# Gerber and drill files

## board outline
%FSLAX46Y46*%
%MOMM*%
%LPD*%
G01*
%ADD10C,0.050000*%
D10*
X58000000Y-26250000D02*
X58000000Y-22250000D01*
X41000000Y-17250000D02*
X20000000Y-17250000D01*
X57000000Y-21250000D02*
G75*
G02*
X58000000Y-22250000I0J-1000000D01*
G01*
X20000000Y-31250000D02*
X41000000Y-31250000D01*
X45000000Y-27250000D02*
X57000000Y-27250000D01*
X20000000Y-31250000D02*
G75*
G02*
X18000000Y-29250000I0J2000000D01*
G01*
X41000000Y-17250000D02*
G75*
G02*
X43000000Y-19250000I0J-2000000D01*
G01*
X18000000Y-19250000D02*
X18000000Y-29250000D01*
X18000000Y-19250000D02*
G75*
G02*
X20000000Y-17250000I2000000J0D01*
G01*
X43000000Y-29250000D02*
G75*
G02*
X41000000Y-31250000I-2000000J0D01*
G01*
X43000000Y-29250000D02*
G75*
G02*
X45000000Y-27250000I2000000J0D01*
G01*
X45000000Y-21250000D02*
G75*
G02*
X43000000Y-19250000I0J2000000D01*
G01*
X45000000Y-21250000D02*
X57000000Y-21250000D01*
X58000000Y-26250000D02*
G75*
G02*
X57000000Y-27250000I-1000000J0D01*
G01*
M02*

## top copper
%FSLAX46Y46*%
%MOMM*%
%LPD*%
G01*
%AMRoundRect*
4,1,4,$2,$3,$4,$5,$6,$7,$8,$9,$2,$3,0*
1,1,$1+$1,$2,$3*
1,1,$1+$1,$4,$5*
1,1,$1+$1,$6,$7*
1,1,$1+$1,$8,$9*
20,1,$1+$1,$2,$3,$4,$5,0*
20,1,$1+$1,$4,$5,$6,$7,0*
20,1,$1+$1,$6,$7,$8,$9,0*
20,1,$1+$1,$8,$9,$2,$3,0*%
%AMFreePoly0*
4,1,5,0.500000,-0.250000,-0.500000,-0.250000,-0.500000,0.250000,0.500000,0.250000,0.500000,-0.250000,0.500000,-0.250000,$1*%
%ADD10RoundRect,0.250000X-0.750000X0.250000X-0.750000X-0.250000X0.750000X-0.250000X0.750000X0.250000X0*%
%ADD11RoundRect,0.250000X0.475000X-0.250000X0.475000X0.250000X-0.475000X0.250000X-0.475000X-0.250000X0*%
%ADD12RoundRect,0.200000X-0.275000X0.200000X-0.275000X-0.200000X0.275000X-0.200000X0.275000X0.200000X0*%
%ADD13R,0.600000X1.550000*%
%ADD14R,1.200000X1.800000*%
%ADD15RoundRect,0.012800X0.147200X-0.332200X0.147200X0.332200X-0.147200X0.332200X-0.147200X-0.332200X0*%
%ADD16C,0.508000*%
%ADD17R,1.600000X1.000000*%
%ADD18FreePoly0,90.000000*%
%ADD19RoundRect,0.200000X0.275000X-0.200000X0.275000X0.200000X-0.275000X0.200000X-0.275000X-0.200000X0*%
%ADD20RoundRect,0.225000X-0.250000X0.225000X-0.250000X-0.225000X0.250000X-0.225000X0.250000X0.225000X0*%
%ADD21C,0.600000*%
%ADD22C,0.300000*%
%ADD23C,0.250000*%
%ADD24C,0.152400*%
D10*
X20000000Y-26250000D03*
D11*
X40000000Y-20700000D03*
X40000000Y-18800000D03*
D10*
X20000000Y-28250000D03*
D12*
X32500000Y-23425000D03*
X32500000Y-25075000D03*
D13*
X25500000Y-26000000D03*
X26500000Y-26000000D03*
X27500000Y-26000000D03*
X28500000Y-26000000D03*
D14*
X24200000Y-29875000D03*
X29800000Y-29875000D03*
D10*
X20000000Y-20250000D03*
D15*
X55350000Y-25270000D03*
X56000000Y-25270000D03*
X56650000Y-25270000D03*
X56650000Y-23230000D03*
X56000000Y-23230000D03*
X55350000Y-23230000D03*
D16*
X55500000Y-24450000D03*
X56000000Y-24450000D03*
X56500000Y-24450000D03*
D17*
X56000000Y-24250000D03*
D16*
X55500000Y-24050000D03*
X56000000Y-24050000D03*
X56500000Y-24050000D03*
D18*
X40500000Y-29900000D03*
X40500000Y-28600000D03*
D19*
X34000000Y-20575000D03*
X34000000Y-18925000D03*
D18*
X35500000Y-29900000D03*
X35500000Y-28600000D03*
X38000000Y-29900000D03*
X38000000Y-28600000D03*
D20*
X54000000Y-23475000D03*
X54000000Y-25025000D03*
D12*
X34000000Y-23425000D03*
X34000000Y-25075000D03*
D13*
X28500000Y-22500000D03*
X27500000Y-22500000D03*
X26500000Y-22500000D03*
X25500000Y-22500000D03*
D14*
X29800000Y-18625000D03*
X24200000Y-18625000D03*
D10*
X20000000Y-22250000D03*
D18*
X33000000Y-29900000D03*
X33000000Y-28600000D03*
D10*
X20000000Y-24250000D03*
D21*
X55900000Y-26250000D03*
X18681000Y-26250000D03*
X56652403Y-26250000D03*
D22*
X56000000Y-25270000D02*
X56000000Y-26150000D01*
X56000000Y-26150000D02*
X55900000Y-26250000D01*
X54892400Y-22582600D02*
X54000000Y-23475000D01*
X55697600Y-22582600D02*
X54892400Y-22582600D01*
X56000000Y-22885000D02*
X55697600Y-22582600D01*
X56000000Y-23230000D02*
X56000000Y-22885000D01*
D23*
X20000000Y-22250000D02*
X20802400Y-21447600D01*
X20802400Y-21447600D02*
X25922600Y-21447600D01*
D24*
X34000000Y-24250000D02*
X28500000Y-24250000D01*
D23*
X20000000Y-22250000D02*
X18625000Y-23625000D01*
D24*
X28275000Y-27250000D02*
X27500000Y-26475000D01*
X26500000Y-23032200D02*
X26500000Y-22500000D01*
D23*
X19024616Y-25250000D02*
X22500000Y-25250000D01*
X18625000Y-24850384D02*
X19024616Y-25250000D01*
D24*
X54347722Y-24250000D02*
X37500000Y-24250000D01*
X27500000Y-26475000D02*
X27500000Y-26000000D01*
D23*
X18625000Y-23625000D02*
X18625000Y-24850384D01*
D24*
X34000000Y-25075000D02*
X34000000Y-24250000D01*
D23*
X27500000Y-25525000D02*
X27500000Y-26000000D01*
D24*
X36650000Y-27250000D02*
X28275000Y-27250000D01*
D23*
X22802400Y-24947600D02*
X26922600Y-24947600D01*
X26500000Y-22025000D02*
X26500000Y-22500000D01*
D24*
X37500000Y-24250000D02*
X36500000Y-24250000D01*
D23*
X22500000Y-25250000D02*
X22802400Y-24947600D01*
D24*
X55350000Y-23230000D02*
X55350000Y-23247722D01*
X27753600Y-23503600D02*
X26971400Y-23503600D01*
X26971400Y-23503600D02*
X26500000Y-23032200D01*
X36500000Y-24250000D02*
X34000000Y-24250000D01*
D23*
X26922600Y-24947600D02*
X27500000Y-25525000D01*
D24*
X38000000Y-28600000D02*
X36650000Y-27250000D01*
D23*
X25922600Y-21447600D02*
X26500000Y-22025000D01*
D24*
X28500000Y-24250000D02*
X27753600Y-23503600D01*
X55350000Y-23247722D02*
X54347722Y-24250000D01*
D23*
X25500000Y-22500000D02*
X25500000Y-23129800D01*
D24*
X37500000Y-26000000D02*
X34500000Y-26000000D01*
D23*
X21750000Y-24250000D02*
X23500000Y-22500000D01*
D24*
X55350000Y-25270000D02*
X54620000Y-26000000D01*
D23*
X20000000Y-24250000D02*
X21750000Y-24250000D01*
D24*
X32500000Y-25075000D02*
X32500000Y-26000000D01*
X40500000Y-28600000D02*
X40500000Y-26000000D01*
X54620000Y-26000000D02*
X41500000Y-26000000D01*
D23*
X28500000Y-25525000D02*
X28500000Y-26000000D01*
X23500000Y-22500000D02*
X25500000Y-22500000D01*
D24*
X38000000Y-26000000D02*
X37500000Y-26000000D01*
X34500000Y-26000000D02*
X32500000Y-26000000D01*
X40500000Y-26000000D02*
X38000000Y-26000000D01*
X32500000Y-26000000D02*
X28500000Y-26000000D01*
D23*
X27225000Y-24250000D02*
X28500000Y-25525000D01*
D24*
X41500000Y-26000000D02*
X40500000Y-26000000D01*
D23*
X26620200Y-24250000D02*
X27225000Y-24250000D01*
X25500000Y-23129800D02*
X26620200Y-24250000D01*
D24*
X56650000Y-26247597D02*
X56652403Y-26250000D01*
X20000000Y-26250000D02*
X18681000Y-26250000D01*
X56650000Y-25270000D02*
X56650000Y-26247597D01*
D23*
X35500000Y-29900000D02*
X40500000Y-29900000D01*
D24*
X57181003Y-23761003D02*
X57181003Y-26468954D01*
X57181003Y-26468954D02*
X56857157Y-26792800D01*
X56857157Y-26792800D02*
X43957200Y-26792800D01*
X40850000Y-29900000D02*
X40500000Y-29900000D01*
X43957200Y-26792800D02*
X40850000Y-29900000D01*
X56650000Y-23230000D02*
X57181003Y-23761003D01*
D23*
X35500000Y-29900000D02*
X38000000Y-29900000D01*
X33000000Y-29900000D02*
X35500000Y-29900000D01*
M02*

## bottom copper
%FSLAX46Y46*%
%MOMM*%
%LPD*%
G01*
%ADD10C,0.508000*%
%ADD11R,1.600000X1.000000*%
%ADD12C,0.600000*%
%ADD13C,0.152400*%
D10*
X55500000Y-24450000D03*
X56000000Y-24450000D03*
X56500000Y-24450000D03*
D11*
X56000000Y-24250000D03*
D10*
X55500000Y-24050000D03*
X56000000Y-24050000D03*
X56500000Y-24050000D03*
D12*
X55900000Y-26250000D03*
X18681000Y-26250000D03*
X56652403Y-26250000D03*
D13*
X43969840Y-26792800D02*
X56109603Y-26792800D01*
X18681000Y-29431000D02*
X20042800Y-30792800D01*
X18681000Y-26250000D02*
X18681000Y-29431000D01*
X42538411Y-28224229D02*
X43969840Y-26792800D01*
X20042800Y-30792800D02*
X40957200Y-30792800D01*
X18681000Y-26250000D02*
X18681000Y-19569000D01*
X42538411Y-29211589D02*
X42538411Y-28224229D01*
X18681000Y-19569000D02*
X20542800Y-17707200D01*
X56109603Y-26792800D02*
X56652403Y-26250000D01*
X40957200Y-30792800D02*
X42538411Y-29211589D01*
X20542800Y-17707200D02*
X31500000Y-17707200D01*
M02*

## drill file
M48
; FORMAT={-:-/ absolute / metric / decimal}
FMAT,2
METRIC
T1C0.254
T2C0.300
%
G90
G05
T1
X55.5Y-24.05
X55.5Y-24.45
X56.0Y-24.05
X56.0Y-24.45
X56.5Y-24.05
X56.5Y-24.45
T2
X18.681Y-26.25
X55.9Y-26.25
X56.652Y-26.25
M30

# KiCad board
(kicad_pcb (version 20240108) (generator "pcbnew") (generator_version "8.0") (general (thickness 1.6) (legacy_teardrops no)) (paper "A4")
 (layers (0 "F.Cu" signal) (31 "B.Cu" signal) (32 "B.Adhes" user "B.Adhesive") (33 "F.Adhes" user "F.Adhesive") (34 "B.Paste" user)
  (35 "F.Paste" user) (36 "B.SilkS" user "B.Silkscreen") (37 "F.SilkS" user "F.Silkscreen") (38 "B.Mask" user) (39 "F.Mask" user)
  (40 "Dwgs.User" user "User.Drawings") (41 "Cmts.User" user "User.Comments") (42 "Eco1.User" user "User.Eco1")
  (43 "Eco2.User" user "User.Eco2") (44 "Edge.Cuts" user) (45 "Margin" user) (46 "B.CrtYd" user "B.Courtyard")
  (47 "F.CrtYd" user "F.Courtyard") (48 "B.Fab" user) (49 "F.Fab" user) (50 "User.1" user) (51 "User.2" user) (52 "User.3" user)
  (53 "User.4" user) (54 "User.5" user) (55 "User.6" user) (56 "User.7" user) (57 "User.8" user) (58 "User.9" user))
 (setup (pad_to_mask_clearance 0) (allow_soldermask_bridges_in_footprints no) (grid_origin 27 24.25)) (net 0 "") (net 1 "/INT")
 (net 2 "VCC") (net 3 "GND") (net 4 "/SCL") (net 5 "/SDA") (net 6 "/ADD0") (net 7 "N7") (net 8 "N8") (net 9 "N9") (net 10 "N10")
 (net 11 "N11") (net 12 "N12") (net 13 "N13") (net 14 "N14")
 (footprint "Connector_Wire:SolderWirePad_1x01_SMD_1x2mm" (layer "F.Cu") (at 20 26.25 -90)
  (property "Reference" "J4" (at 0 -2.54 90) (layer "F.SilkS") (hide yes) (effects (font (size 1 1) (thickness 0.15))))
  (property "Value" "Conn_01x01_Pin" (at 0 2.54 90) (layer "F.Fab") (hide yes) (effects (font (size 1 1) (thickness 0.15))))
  (pad "1" smd roundrect (at 0 0 270) (size 1 2) (layers "F.Cu" "F.Paste" "F.Mask") (roundrect_rratio 0.25) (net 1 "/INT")))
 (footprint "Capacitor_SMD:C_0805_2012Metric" (layer "F.Cu") (at 40 19.75 90)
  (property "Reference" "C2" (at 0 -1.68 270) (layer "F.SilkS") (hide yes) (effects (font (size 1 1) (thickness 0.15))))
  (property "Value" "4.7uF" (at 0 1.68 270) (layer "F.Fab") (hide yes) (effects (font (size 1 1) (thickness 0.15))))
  (pad "1" smd roundrect (at -0.95 0 90) (size 1 1.45) (layers "F.Cu" "F.Paste" "F.Mask") (roundrect_rratio 0.25) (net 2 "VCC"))
  (pad "2" smd roundrect (at 0.95 0 90) (size 1 1.45) (layers "F.Cu" "F.Paste" "F.Mask") (roundrect_rratio 0.25) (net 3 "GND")))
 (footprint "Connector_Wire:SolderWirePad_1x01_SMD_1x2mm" (layer "F.Cu") (at 20 28.25 -90)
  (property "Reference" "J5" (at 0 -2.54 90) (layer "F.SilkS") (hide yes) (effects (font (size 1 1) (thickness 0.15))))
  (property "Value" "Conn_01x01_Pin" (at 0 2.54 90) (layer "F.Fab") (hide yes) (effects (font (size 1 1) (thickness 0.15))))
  (pad "1" smd roundrect (at 0 0 270) (size 1 2) (layers "F.Cu" "F.Paste" "F.Mask") (roundrect_rratio 0.25) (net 3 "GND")))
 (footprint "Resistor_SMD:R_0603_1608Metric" (layer "F.Cu") (at 32.5 24.25 -90)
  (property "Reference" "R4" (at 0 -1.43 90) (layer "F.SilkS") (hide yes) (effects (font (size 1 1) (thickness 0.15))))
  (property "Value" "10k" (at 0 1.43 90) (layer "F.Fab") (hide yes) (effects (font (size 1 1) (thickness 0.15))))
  (pad "1" smd roundrect (at -0.825 0 270) (size 0.8 0.95) (layers "F.Cu" "F.Paste" "F.Mask") (roundrect_rratio 0.25) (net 2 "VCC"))
  (pad "2" smd roundrect (at 0.825 0 270) (size 0.8 0.95) (layers "F.Cu" "F.Paste" "F.Mask") (roundrect_rratio 0.25) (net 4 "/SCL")))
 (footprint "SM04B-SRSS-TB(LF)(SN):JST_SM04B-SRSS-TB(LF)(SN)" (layer "F.Cu") (at 27 26)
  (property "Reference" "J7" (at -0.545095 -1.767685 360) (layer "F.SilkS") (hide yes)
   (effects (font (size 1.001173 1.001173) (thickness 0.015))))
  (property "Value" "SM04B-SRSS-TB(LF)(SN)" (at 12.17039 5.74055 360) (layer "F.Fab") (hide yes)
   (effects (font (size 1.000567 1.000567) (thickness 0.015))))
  (pad "1" smd rect (at -1.5 0) (size 0.6 1.55) (layers "F.Cu" "F.Paste" "F.Mask") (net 3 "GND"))
  (pad "2" smd rect (at -0.5 0) (size 0.6 1.55) (layers "F.Cu" "F.Paste" "F.Mask") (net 2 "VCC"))
  (pad "3" smd rect (at 0.5 0) (size 0.6 1.55) (layers "F.Cu" "F.Paste" "F.Mask") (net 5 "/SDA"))
  (pad "4" smd rect (at 1.5 0) (size 0.6 1.55) (layers "F.Cu" "F.Paste" "F.Mask") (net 4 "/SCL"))
  (pad "S1" smd rect (at -2.8 3.875) (size 1.2 1.8) (layers "F.Cu" "F.Paste" "F.Mask") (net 3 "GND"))
  (pad "S2" smd rect (at 2.8 3.875) (size 1.2 1.8) (layers "F.Cu" "F.Paste" "F.Mask") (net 3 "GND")))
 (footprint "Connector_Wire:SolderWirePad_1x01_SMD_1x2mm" (layer "F.Cu") (at 20 20.25 -90)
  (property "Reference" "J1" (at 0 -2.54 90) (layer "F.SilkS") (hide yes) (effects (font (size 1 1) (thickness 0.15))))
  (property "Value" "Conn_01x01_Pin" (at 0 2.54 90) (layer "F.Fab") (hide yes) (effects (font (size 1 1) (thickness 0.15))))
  (pad "1" smd roundrect (at 0 0 270) (size 1 2) (layers "F.Cu" "F.Paste" "F.Mask") (roundrect_rratio 0.25) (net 2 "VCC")))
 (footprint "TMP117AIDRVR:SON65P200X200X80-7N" (layer "F.Cu") (at 56 24.25 90)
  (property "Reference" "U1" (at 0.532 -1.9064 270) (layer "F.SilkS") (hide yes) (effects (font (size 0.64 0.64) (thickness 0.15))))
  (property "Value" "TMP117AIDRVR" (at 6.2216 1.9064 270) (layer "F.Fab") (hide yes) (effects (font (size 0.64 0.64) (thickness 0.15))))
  (pad "1" smd roundrect (at -1.02 -0.65 90) (size 0.69 0.32) (layers "F.Cu" "F.Paste" "F.Mask") (roundrect_rratio 0.04) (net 4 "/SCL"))
  (pad "2" smd roundrect (at -1.02 0 90) (size 0.69 0.32) (layers "F.Cu" "F.Paste" "F.Mask") (roundrect_rratio 0.04) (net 3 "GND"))
  (pad "3" smd roundrect (at -1.02 0.65 90) (size 0.69 0.32) (layers "F.Cu" "F.Paste" "F.Mask") (roundrect_rratio 0.04) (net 1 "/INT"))
  (pad "4" smd roundrect (at 1.02 0.65 90) (size 0.69 0.32) (layers "F.Cu" "F.Paste" "F.Mask") (roundrect_rratio 0.04) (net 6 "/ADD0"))
  (pad "5" smd roundrect (at 1.02 0 90) (size 0.69 0.32) (layers "F.Cu" "F.Paste" "F.Mask") (roundrect_rratio 0.04) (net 2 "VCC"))
  (pad "6" smd roundrect (at 1.02 -0.65 90) (size 0.69 0.32) (layers "F.Cu" "F.Paste" "F.Mask") (roundrect_rratio 0.04) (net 5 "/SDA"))
  (pad "7" thru_hole circle (at -0.2 -0.5 180) (size 0.508 0.508) (drill 0.254) (layers "*.Cu" "*.Mask") (remove_unused_layers no)
   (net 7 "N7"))
  (pad "7" thru_hole circle (at -0.2 0 180) (size 0.508 0.508) (drill 0.254) (layers "*.Cu" "*.Mask") (remove_unused_layers no) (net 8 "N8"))
  (pad "7" thru_hole circle (at -0.2 0.5 180) (size 0.508 0.508) (drill 0.254) (layers "*.Cu" "*.Mask") (remove_unused_layers no)
   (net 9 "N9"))
  (pad "7" smd rect (at 0 0 180) (size 1.6 1) (layers "F.Cu" "F.Mask") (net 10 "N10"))
  (pad "7" smd rect (at 0 0 180) (size 1.6 1) (layers "B.Cu" "B.Mask") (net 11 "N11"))
  (pad "7" thru_hole circle (at 0.2 -0.5 180) (size 0.508 0.508) (drill 0.254) (layers "*.Cu" "*.Mask") (remove_unused_layers no)
   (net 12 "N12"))
  (pad "7" thru_hole circle (at 0.2 0 180) (size 0.508 0.508) (drill 0.254) (layers "*.Cu" "*.Mask") (remove_unused_layers no)
   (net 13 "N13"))
  (pad "7" thru_hole circle (at 0.2 0.5 180) (size 0.508 0.508) (drill 0.254) (layers "*.Cu" "*.Mask") (remove_unused_layers no)
   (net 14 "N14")))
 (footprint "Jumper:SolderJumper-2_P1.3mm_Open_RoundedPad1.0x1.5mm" (layer "F.Cu") (at 40.5 29.25 90)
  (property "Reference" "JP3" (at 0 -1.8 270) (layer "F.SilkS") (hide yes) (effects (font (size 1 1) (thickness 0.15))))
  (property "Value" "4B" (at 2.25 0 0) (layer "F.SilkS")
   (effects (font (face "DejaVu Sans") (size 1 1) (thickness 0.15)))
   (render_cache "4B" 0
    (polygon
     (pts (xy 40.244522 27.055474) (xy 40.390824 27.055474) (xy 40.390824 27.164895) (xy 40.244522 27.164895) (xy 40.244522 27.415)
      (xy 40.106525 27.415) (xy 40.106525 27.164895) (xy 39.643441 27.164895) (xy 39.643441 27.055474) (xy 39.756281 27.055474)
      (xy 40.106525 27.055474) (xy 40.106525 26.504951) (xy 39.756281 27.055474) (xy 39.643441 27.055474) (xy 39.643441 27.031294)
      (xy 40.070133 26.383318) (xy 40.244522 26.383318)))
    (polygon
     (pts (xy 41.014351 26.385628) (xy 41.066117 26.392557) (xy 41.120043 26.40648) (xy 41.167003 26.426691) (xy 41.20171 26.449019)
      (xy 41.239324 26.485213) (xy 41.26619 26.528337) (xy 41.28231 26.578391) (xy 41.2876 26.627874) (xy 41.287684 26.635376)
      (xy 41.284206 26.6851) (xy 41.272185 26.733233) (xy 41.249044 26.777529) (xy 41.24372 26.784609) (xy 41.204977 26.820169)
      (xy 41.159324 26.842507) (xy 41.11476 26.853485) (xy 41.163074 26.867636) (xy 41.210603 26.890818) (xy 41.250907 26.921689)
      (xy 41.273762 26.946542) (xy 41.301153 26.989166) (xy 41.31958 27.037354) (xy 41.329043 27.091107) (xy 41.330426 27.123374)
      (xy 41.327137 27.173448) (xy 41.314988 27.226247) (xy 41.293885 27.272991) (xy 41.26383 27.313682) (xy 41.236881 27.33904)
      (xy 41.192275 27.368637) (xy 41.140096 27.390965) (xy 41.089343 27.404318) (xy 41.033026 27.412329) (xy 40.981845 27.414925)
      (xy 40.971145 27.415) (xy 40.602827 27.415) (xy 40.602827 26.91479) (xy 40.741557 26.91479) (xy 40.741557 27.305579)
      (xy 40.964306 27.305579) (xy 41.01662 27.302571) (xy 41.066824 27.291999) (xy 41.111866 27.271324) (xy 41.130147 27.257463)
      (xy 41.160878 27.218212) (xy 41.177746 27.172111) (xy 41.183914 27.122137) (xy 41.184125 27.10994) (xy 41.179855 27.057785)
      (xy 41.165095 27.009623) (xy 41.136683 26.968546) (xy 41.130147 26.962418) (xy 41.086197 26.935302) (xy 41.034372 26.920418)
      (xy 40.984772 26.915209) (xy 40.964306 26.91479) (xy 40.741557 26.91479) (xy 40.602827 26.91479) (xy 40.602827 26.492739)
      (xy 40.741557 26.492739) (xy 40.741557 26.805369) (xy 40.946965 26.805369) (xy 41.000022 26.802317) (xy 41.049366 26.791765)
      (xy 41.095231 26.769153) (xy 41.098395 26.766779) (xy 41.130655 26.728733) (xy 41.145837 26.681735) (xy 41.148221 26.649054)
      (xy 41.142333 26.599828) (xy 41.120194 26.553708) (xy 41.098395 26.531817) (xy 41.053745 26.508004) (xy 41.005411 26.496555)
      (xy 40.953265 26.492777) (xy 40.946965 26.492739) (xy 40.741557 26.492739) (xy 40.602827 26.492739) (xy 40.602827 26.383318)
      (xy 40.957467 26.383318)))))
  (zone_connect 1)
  (pad "1" smd custom (at -0.65 0 90) (size 1 0.5) (layers "F.Cu" "F.Mask") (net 6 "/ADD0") (zone_connect 2) (thermal_bridge_angle 45)
   (options (clearance outline) (anchor rect)) (primitives))
  (pad "2" smd custom (at 0.65 0 90) (size 1 0.5) (layers "F.Cu" "F.Mask") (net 4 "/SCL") (zone_connect 2) (thermal_bridge_angle 45)
   (options (clearance outline) (anchor rect)) (primitives)))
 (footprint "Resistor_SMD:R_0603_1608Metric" (layer "F.Cu") (at 34 19.75 90)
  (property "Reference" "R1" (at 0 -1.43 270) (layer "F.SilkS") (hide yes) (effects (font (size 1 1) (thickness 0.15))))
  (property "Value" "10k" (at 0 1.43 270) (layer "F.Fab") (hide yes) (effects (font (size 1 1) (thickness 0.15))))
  (pad "1" smd roundrect (at -0.825 0 90) (size 0.8 0.95) (layers "F.Cu" "F.Paste" "F.Mask") (roundrect_rratio 0.25) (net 2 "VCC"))
  (pad "2" smd roundrect (at 0.825 0 90) (size 0.8 0.95) (layers "F.Cu" "F.Paste" "F.Mask") (roundrect_rratio 0.25) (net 1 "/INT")))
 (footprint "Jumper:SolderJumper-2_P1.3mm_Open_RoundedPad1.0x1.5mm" (layer "F.Cu") (at 35.5 29.25 90)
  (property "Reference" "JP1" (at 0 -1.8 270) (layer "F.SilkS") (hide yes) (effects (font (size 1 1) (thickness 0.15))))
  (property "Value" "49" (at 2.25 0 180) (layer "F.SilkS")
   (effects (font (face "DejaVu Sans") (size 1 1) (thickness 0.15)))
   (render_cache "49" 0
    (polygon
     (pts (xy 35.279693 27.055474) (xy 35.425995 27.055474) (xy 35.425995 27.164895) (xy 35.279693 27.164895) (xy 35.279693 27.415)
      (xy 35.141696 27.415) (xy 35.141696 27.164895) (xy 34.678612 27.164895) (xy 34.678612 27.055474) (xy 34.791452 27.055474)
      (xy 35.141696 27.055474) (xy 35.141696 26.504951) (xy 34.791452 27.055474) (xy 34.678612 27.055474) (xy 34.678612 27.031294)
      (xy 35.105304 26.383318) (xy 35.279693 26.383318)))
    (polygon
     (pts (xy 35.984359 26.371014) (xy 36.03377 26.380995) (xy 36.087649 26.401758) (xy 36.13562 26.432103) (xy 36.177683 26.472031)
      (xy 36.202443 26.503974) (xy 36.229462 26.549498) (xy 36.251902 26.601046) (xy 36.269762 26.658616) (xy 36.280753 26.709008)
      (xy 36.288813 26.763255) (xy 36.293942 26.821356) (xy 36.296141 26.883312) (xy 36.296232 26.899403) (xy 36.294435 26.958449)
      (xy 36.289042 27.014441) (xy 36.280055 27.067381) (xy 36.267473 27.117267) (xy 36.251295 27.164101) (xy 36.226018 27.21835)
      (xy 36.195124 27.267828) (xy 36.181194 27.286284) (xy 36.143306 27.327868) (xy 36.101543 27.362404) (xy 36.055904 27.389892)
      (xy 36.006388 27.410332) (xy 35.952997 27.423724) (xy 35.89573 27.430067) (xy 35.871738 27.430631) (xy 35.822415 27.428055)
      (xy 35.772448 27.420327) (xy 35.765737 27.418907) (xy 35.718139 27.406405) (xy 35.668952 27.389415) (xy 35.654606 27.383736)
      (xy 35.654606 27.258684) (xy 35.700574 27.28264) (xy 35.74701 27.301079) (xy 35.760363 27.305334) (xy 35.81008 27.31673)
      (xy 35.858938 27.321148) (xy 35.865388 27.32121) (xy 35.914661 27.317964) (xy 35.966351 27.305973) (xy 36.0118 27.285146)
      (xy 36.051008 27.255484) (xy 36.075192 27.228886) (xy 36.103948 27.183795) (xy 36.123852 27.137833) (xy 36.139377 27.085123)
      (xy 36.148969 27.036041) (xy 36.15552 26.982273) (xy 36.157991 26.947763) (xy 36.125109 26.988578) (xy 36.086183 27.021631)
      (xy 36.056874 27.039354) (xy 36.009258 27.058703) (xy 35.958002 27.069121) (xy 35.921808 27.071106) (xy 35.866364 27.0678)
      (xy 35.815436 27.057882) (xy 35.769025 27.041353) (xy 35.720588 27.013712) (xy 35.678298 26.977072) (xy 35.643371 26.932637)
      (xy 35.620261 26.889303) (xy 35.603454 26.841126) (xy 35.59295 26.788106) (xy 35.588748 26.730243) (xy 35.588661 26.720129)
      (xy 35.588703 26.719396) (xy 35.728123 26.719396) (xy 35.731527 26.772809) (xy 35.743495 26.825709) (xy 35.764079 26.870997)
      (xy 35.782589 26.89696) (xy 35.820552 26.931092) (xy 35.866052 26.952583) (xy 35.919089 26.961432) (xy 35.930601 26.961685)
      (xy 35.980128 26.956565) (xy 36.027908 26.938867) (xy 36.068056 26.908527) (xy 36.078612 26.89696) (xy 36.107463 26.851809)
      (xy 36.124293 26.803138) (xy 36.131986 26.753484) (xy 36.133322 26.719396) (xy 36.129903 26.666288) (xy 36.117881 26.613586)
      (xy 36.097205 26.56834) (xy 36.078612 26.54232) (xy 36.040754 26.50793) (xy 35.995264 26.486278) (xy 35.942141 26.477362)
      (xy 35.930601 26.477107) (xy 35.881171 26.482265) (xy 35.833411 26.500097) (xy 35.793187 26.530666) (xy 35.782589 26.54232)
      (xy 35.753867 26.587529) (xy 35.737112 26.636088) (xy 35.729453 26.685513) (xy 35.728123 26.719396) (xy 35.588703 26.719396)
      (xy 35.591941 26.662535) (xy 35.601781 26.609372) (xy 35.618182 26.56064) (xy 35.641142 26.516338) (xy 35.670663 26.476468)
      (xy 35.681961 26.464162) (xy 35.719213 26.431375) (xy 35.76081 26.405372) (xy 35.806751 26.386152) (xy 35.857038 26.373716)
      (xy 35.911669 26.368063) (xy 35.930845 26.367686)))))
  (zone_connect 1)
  (pad "1" smd custom (at -0.65 0 90) (size 1 0.5) (layers "F.Cu" "F.Mask") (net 6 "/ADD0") (zone_connect 2) (thermal_bridge_angle 45)
   (options (clearance outline) (anchor rect)) (primitives))
  (pad "2" smd custom (at 0.65 0 90) (size 1 0.5) (layers "F.Cu" "F.Mask") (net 2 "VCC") (zone_connect 2) (thermal_bridge_angle 45)
   (options (clearance outline) (anchor rect)) (primitives)))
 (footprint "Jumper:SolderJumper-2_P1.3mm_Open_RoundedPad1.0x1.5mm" (layer "F.Cu") (at 38 29.25 90)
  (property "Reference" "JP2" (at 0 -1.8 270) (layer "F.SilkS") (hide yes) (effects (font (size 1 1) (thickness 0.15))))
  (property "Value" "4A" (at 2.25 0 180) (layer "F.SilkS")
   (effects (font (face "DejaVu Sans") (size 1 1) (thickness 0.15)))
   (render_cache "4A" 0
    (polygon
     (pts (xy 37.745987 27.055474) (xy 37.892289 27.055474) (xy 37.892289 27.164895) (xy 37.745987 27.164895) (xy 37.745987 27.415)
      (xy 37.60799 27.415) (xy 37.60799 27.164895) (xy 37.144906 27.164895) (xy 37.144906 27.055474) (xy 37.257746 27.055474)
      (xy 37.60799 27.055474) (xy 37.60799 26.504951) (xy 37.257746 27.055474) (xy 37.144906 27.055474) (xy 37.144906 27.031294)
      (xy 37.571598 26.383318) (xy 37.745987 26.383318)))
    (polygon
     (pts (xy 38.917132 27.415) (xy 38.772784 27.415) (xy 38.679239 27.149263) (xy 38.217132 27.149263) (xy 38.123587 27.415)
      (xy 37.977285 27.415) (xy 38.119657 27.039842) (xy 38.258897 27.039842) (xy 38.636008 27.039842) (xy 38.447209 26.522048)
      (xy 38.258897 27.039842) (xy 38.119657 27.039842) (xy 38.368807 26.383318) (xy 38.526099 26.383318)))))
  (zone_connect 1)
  (pad "1" smd custom (at -0.65 0 90) (size 1 0.5) (layers "F.Cu" "F.Mask") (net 6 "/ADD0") (zone_connect 2) (thermal_bridge_angle 45)
   (options (clearance outline) (anchor rect)) (primitives))
  (pad "2" smd custom (at 0.65 0 90) (size 1 0.5) (layers "F.Cu" "F.Mask") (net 5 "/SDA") (zone_connect 2) (thermal_bridge_angle 45)
   (options (clearance outline) (anchor rect)) (primitives)))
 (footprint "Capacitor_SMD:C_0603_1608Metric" (layer "F.Cu") (at 54 24.25 -90)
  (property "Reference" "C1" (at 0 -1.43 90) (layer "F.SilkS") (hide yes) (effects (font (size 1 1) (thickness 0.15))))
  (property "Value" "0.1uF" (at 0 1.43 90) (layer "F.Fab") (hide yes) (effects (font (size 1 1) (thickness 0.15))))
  (pad "1" smd roundrect (at -0.775 0 270) (size 0.9 0.95) (layers "F.Cu" "F.Paste" "F.Mask") (roundrect_rratio 0.25) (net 2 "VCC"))
  (pad "2" smd roundrect (at 0.775 0 270) (size 0.9 0.95) (layers "F.Cu" "F.Paste" "F.Mask") (roundrect_rratio 0.25) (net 3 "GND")))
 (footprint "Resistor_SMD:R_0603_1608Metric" (layer "F.Cu") (at 34 24.25 -90)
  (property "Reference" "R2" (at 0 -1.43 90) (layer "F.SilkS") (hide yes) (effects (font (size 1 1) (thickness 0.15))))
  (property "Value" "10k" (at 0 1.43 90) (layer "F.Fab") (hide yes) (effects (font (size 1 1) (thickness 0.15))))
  (pad "1" smd roundrect (at -0.825 0 270) (size 0.8 0.95) (layers "F.Cu" "F.Paste" "F.Mask") (roundrect_rratio 0.25) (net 2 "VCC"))
  (pad "2" smd roundrect (at 0.825 0 270) (size 0.8 0.95) (layers "F.Cu" "F.Paste" "F.Mask") (roundrect_rratio 0.25) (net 5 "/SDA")))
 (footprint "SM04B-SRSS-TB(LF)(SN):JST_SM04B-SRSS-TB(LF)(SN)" (layer "F.Cu") (at 27 22.5 180)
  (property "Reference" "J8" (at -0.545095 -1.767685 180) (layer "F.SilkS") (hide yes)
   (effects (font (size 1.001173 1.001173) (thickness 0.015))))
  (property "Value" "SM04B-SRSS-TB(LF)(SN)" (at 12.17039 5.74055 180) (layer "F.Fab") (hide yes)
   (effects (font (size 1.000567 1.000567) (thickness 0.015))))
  (pad "1" smd rect (at -1.5 0 180) (size 0.6 1.55) (layers "F.Cu" "F.Paste" "F.Mask") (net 3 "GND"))
  (pad "2" smd rect (at -0.5 0 180) (size 0.6 1.55) (layers "F.Cu" "F.Paste" "F.Mask") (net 2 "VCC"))
  (pad "3" smd rect (at 0.5 0 180) (size 0.6 1.55) (layers "F.Cu" "F.Paste" "F.Mask") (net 5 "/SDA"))
  (pad "4" smd rect (at 1.5 0 180) (size 0.6 1.55) (layers "F.Cu" "F.Paste" "F.Mask") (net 4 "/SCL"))
  (pad "S1" smd rect (at -2.8 3.875 180) (size 1.2 1.8) (layers "F.Cu" "F.Paste" "F.Mask") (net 3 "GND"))
  (pad "S2" smd rect (at 2.8 3.875 180) (size 1.2 1.8) (layers "F.Cu" "F.Paste" "F.Mask") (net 3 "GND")))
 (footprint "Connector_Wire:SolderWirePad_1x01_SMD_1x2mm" (layer "F.Cu") (at 20 22.25 -90)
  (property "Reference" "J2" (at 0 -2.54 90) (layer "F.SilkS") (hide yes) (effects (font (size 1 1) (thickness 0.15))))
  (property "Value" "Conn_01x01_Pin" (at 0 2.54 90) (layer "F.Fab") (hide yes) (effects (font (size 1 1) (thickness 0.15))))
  (pad "1" smd roundrect (at 0 0 270) (size 1 2) (layers "F.Cu" "F.Paste" "F.Mask") (roundrect_rratio 0.25) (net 5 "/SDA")))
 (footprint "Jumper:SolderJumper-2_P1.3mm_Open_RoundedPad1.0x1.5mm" (layer "F.Cu") (at 33 29.25 90)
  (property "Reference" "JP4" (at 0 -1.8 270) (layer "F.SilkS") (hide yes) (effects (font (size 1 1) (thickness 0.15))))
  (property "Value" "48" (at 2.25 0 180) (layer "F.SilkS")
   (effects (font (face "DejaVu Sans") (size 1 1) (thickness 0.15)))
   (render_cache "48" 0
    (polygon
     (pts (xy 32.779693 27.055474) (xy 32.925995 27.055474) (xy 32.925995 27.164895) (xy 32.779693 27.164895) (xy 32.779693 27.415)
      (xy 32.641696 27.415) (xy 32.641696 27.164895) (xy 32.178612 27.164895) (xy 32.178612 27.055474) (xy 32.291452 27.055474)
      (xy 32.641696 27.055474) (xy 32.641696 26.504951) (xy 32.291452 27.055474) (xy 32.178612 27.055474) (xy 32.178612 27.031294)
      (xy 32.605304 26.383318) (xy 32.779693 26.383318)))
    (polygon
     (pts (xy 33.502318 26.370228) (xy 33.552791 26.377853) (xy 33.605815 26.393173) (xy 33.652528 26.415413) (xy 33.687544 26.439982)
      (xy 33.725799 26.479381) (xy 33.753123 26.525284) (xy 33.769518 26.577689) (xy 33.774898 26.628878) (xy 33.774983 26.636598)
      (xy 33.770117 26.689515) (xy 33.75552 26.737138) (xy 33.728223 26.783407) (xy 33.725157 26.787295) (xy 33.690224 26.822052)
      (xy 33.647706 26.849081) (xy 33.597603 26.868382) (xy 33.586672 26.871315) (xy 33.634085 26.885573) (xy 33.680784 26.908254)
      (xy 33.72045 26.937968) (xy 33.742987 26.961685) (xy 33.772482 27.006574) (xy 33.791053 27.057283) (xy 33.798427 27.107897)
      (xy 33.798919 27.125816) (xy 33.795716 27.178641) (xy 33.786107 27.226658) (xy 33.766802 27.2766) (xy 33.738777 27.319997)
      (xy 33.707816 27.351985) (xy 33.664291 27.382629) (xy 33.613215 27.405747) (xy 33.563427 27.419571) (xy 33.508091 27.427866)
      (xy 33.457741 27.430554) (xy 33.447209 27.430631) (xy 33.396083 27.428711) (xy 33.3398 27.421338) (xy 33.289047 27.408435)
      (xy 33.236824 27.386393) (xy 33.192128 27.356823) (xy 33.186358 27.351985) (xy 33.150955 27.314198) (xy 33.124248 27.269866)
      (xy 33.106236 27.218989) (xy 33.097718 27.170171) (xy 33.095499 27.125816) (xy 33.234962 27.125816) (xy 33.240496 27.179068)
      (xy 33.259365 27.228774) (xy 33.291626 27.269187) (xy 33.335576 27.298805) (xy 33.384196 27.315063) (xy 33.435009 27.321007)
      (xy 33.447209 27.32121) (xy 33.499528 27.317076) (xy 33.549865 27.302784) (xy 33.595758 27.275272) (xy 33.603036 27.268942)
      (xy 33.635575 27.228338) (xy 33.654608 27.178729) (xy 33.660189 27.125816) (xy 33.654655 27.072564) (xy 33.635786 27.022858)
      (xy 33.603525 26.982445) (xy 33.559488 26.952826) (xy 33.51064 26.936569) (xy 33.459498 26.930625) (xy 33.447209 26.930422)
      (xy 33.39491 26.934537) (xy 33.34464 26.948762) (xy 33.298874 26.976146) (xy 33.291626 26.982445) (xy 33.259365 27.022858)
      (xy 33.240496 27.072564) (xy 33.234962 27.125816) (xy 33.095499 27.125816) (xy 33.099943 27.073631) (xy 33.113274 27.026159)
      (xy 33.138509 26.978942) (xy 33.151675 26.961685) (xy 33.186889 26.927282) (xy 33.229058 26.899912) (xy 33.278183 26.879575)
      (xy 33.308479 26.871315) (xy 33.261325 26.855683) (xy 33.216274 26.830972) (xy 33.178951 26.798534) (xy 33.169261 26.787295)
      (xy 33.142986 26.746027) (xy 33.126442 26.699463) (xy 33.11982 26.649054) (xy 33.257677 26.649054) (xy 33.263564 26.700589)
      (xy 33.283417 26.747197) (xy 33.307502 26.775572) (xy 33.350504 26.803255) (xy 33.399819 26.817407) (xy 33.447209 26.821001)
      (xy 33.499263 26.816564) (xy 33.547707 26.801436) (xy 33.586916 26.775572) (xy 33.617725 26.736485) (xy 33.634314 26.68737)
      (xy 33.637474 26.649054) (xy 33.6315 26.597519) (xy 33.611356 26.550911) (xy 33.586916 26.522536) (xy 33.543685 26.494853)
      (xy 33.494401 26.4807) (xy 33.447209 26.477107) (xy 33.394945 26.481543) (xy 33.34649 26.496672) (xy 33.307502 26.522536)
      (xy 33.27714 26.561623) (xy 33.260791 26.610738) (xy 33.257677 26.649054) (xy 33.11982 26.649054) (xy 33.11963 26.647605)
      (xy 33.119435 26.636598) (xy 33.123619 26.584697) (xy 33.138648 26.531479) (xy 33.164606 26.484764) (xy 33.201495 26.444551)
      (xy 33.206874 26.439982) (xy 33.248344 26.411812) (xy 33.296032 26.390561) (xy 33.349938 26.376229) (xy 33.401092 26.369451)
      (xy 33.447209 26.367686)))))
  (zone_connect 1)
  (pad "1" smd custom (at -0.65 0 90) (size 1 0.5) (layers "F.Cu" "F.Mask") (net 6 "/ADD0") (zone_connect 2) (thermal_bridge_angle 45)
   (options (clearance outline) (anchor rect)) (primitives))
  (pad "2" smd custom (at 0.65 0 90) (size 1 0.5) (layers "F.Cu" "F.Mask") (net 3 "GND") (zone_connect 2) (thermal_bridge_angle 45)
   (options (clearance outline) (anchor rect)) (primitives)))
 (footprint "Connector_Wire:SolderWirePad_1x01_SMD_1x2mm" (layer "F.Cu") (at 20 24.25 -90)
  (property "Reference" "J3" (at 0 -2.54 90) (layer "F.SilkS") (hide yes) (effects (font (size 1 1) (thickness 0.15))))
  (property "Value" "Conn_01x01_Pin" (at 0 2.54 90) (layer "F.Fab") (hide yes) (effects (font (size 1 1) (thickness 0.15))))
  (pad "1" smd roundrect (at 0 0 270) (size 1 2) (layers "F.Cu" "F.Paste" "F.Mask") (roundrect_rratio 0.25) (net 4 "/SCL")))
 (gr_line (start 58 26.25) (end 58 22.25) (stroke (width 0.05) (type default)) (layer "Edge.Cuts"))
 (gr_line (start 41 17.25) (end 20 17.25) (stroke (width 0.05) (type default)) (layer "Edge.Cuts"))
 (gr_arc (start 57 21.25) (mid 57.707107 21.542893) (end 58 22.25) (stroke (width 0.05) (type default)) (layer "Edge.Cuts"))
 (gr_line (start 20 31.25) (end 41 31.25) (stroke (width 0.05) (type default)) (layer "Edge.Cuts"))
 (gr_line (start 45 27.25) (end 57 27.25) (stroke (width 0.05) (type default)) (layer "Edge.Cuts"))
 (gr_arc (start 20 31.25) (mid 18.585786 30.664214) (end 18 29.25) (stroke (width 0.05) (type default)) (layer "Edge.Cuts"))
 (gr_arc (start 41 17.25) (mid 42.414214 17.835786) (end 43 19.25) (stroke (width 0.05) (type default)) (layer "Edge.Cuts"))
 (gr_line (start 18 19.25) (end 18 29.25) (stroke (width 0.05) (type default)) (layer "Edge.Cuts"))
 (gr_arc (start 18 19.25) (mid 18.585786 17.835786) (end 20 17.25) (stroke (width 0.05) (type default)) (layer "Edge.Cuts"))
 (gr_arc (start 43 29.25) (mid 42.414214 30.664214) (end 41 31.25) (stroke (width 0.05) (type default)) (layer "Edge.Cuts"))
 (gr_arc (start 43 29.25) (mid 43.585786 27.835786) (end 45 27.25) (stroke (width 0.05) (type default)) (layer "Edge.Cuts"))
 (gr_arc (start 45 21.25) (mid 43.585786 20.664214) (end 43 19.25) (stroke (width 0.05) (type default)) (layer "Edge.Cuts"))
 (gr_line (start 45 21.25) (end 57 21.25) (stroke (width 0.05) (type default)) (layer "Edge.Cuts"))
 (gr_arc (start 58 26.25) (mid 57.707107 26.957107) (end 57 27.25) (stroke (width 0.05) (type default)) (layer "Edge.Cuts"))
 (segment (start 56 25.27) (end 56 26.15) (width 0.3) (layer "F.Cu") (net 3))
 (segment (start 56 26.15) (end 55.9 26.25) (width 0.3) (layer "F.Cu") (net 3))
 (via (at 55.9 26.25) (size 0.6) (drill 0.3) (layers "F.Cu" "B.Cu") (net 3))
 (segment (start 54.8924 22.5826) (end 54 23.475) (width 0.3) (layer "F.Cu") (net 2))
 (segment (start 55.6976 22.5826) (end 54.8924 22.5826) (width 0.3) (layer "F.Cu") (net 2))
 (segment (start 56 22.885) (end 55.6976 22.5826) (width 0.3) (layer "F.Cu") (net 2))
 (segment (start 56 23.23) (end 56 22.885) (width 0.3) (layer "F.Cu") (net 2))
 (segment (start 20 22.25) (end 20.8024 21.4476) (width 0.25) (layer "F.Cu") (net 5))
 (segment (start 20.8024 21.4476) (end 25.9226 21.4476) (width 0.25) (layer "F.Cu") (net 5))
 (segment (start 34 24.25) (end 28.5 24.25) (width 0.1524) (layer "F.Cu") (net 5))
 (segment (start 20 22.25) (end 18.625 23.625) (width 0.25) (layer "F.Cu") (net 5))
 (segment (start 28.275 27.25) (end 27.5 26.475) (width 0.1524) (layer "F.Cu") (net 5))
 (segment (start 26.5 23.0322) (end 26.5 22.5) (width 0.1524) (layer "F.Cu") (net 5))
 (segment (start 19.024616 25.25) (end 22.5 25.25) (width 0.25) (layer "F.Cu") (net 5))
 (segment (start 18.625 24.850384) (end 19.024616 25.25) (width 0.25) (layer "F.Cu") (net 5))
 (segment (start 54.347722 24.25) (end 37.5 24.25) (width 0.1524) (layer "F.Cu") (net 5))
 (segment (start 27.5 26.475) (end 27.5 26) (width 0.1524) (layer "F.Cu") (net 5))
 (segment (start 18.625 23.625) (end 18.625 24.850384) (width 0.25) (layer "F.Cu") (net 5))
 (segment (start 34 25.075) (end 34 24.25) (width 0.1524) (layer "F.Cu") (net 5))
 (segment (start 27.5 25.525) (end 27.5 26) (width 0.25) (layer "F.Cu") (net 5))
 (segment (start 36.65 27.25) (end 28.275 27.25) (width 0.1524) (layer "F.Cu") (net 5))
 (segment (start 22.8024 24.9476) (end 26.9226 24.9476) (width 0.25) (layer "F.Cu") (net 5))
 (segment (start 26.5 22.025) (end 26.5 22.5) (width 0.25) (layer "F.Cu") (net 5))
 (segment (start 37.5 24.25) (end 36.5 24.25) (width 0.1524) (layer "F.Cu") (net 5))
 (segment (start 22.5 25.25) (end 22.8024 24.9476) (width 0.25) (layer "F.Cu") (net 5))
 (segment (start 55.35 23.23) (end 55.35 23.247722) (width 0.1524) (layer "F.Cu") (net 5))
 (segment (start 27.7536 23.5036) (end 26.9714 23.5036) (width 0.1524) (layer "F.Cu") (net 5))
 (segment (start 26.9714 23.5036) (end 26.5 23.0322) (width 0.1524) (layer "F.Cu") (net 5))
 (segment (start 36.5 24.25) (end 34 24.25) (width 0.1524) (layer "F.Cu") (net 5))
 (segment (start 26.9226 24.9476) (end 27.5 25.525) (width 0.25) (layer "F.Cu") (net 5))
 (segment (start 38 28.6) (end 36.65 27.25) (width 0.1524) (layer "F.Cu") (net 5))
 (segment (start 25.9226 21.4476) (end 26.5 22.025) (width 0.25) (layer "F.Cu") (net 5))
 (segment (start 28.5 24.25) (end 27.7536 23.5036) (width 0.1524) (layer "F.Cu") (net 5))
 (segment (start 55.35 23.247722) (end 54.347722 24.25) (width 0.1524) (layer "F.Cu") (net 5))
 (segment (start 25.5 22.5) (end 25.5 23.1298) (width 0.25) (layer "F.Cu") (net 4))
 (segment (start 37.5 26) (end 34.5 26) (width 0.1524) (layer "F.Cu") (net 4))
 (segment (start 21.75 24.25) (end 23.5 22.5) (width 0.25) (layer "F.Cu") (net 4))
 (segment (start 55.35 25.27) (end 54.62 26) (width 0.1524) (layer "F.Cu") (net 4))
 (segment (start 20 24.25) (end 21.75 24.25) (width 0.25) (layer "F.Cu") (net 4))
 (segment (start 32.5 25.075) (end 32.5 26) (width 0.1524) (layer "F.Cu") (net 4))
 (segment (start 40.5 28.6) (end 40.5 26) (width 0.1524) (layer "F.Cu") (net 4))
 (segment (start 54.62 26) (end 41.5 26) (width 0.1524) (layer "F.Cu") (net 4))
 (segment (start 28.5 25.525) (end 28.5 26) (width 0.25) (layer "F.Cu") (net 4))
 (segment (start 23.5 22.5) (end 25.5 22.5) (width 0.25) (layer "F.Cu") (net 4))
 (segment (start 38 26) (end 37.5 26) (width 0.1524) (layer "F.Cu") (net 4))
 (segment (start 34.5 26) (end 32.5 26) (width 0.1524) (layer "F.Cu") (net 4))
 (segment (start 40.5 26) (end 38 26) (width 0.1524) (layer "F.Cu") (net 4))
 (segment (start 32.5 26) (end 28.5 26) (width 0.1524) (layer "F.Cu") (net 4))
 (segment (start 27.225 24.25) (end 28.5 25.525) (width 0.25) (layer "F.Cu") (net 4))
 (segment (start 41.5 26) (end 40.5 26) (width 0.1524) (layer "F.Cu") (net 4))
 (segment (start 26.6202 24.25) (end 27.225 24.25) (width 0.25) (layer "F.Cu") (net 4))
 (segment (start 25.5 23.1298) (end 26.6202 24.25) (width 0.25) (layer "F.Cu") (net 4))
 (segment (start 56.65 26.247597) (end 56.652403 26.25) (width 0.1524) (layer "F.Cu") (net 1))
 (segment (start 20 26.25) (end 18.681 26.25) (width 0.1524) (layer "F.Cu") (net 1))
 (segment (start 56.65 25.27) (end 56.65 26.247597) (width 0.1524) (layer "F.Cu") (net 1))
 (via (at 18.681 26.25) (size 0.6) (drill 0.3) (layers "F.Cu" "B.Cu") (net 1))
 (via (at 56.652403 26.25) (size 0.6) (drill 0.3) (layers "F.Cu" "B.Cu") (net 1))
 (segment (start 43.96984 26.7928) (end 56.109603 26.7928) (width 0.1524) (layer "B.Cu") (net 1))
 (segment (start 18.681 29.431) (end 20.0428 30.7928) (width 0.1524) (layer "B.Cu") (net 1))
 (segment (start 18.681 26.25) (end 18.681 29.431) (width 0.1524) (layer "B.Cu") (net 1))
 (segment (start 42.538411 28.224229) (end 43.96984 26.7928) (width 0.1524) (layer "B.Cu") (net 1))
 (segment (start 20.0428 30.7928) (end 40.9572 30.7928) (width 0.1524) (layer "B.Cu") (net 1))
 (segment (start 18.681 26.25) (end 18.681 19.569) (width 0.1524) (layer "B.Cu") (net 1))
 (segment (start 42.538411 29.211589) (end 42.538411 28.224229) (width 0.1524) (layer "B.Cu") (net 1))
 (segment (start 18.681 19.569) (end 20.5428 17.7072) (width 0.1524) (layer "B.Cu") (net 1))
 (segment (start 56.109603 26.7928) (end 56.652403 26.25) (width 0.1524) (layer "B.Cu") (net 1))
 (segment (start 40.9572 30.7928) (end 42.538411 29.211589) (width 0.1524) (layer "B.Cu") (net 1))
 (segment (start 20.5428 17.7072) (end 31.5 17.7072) (width 0.1524) (layer "B.Cu") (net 1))
 (segment (start 35.5 29.9) (end 40.5 29.9) (width 0.25) (layer "F.Cu") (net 6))
 (segment (start 57.181003 23.761003) (end 57.181003 26.468954) (width 0.1524) (layer "F.Cu") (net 6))
 (segment (start 57.181003 26.468954) (end 56.857157 26.7928) (width 0.1524) (layer "F.Cu") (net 6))
 (segment (start 56.857157 26.7928) (end 43.9572 26.7928) (width 0.1524) (layer "F.Cu") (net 6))
 (segment (start 40.85 29.9) (end 40.5 29.9) (width 0.1524) (layer "F.Cu") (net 6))
 (segment (start 43.9572 26.7928) (end 40.85 29.9) (width 0.1524) (layer "F.Cu") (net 6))
 (segment (start 56.65 23.23) (end 57.181003 23.761003) (width 0.1524) (layer "F.Cu") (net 6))
 (segment (start 35.5 29.9) (end 38 29.9) (width 0.25) (layer "F.Cu") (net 6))
 (segment (start 33 29.9) (end 35.5 29.9) (width 0.25) (layer "F.Cu") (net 6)))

